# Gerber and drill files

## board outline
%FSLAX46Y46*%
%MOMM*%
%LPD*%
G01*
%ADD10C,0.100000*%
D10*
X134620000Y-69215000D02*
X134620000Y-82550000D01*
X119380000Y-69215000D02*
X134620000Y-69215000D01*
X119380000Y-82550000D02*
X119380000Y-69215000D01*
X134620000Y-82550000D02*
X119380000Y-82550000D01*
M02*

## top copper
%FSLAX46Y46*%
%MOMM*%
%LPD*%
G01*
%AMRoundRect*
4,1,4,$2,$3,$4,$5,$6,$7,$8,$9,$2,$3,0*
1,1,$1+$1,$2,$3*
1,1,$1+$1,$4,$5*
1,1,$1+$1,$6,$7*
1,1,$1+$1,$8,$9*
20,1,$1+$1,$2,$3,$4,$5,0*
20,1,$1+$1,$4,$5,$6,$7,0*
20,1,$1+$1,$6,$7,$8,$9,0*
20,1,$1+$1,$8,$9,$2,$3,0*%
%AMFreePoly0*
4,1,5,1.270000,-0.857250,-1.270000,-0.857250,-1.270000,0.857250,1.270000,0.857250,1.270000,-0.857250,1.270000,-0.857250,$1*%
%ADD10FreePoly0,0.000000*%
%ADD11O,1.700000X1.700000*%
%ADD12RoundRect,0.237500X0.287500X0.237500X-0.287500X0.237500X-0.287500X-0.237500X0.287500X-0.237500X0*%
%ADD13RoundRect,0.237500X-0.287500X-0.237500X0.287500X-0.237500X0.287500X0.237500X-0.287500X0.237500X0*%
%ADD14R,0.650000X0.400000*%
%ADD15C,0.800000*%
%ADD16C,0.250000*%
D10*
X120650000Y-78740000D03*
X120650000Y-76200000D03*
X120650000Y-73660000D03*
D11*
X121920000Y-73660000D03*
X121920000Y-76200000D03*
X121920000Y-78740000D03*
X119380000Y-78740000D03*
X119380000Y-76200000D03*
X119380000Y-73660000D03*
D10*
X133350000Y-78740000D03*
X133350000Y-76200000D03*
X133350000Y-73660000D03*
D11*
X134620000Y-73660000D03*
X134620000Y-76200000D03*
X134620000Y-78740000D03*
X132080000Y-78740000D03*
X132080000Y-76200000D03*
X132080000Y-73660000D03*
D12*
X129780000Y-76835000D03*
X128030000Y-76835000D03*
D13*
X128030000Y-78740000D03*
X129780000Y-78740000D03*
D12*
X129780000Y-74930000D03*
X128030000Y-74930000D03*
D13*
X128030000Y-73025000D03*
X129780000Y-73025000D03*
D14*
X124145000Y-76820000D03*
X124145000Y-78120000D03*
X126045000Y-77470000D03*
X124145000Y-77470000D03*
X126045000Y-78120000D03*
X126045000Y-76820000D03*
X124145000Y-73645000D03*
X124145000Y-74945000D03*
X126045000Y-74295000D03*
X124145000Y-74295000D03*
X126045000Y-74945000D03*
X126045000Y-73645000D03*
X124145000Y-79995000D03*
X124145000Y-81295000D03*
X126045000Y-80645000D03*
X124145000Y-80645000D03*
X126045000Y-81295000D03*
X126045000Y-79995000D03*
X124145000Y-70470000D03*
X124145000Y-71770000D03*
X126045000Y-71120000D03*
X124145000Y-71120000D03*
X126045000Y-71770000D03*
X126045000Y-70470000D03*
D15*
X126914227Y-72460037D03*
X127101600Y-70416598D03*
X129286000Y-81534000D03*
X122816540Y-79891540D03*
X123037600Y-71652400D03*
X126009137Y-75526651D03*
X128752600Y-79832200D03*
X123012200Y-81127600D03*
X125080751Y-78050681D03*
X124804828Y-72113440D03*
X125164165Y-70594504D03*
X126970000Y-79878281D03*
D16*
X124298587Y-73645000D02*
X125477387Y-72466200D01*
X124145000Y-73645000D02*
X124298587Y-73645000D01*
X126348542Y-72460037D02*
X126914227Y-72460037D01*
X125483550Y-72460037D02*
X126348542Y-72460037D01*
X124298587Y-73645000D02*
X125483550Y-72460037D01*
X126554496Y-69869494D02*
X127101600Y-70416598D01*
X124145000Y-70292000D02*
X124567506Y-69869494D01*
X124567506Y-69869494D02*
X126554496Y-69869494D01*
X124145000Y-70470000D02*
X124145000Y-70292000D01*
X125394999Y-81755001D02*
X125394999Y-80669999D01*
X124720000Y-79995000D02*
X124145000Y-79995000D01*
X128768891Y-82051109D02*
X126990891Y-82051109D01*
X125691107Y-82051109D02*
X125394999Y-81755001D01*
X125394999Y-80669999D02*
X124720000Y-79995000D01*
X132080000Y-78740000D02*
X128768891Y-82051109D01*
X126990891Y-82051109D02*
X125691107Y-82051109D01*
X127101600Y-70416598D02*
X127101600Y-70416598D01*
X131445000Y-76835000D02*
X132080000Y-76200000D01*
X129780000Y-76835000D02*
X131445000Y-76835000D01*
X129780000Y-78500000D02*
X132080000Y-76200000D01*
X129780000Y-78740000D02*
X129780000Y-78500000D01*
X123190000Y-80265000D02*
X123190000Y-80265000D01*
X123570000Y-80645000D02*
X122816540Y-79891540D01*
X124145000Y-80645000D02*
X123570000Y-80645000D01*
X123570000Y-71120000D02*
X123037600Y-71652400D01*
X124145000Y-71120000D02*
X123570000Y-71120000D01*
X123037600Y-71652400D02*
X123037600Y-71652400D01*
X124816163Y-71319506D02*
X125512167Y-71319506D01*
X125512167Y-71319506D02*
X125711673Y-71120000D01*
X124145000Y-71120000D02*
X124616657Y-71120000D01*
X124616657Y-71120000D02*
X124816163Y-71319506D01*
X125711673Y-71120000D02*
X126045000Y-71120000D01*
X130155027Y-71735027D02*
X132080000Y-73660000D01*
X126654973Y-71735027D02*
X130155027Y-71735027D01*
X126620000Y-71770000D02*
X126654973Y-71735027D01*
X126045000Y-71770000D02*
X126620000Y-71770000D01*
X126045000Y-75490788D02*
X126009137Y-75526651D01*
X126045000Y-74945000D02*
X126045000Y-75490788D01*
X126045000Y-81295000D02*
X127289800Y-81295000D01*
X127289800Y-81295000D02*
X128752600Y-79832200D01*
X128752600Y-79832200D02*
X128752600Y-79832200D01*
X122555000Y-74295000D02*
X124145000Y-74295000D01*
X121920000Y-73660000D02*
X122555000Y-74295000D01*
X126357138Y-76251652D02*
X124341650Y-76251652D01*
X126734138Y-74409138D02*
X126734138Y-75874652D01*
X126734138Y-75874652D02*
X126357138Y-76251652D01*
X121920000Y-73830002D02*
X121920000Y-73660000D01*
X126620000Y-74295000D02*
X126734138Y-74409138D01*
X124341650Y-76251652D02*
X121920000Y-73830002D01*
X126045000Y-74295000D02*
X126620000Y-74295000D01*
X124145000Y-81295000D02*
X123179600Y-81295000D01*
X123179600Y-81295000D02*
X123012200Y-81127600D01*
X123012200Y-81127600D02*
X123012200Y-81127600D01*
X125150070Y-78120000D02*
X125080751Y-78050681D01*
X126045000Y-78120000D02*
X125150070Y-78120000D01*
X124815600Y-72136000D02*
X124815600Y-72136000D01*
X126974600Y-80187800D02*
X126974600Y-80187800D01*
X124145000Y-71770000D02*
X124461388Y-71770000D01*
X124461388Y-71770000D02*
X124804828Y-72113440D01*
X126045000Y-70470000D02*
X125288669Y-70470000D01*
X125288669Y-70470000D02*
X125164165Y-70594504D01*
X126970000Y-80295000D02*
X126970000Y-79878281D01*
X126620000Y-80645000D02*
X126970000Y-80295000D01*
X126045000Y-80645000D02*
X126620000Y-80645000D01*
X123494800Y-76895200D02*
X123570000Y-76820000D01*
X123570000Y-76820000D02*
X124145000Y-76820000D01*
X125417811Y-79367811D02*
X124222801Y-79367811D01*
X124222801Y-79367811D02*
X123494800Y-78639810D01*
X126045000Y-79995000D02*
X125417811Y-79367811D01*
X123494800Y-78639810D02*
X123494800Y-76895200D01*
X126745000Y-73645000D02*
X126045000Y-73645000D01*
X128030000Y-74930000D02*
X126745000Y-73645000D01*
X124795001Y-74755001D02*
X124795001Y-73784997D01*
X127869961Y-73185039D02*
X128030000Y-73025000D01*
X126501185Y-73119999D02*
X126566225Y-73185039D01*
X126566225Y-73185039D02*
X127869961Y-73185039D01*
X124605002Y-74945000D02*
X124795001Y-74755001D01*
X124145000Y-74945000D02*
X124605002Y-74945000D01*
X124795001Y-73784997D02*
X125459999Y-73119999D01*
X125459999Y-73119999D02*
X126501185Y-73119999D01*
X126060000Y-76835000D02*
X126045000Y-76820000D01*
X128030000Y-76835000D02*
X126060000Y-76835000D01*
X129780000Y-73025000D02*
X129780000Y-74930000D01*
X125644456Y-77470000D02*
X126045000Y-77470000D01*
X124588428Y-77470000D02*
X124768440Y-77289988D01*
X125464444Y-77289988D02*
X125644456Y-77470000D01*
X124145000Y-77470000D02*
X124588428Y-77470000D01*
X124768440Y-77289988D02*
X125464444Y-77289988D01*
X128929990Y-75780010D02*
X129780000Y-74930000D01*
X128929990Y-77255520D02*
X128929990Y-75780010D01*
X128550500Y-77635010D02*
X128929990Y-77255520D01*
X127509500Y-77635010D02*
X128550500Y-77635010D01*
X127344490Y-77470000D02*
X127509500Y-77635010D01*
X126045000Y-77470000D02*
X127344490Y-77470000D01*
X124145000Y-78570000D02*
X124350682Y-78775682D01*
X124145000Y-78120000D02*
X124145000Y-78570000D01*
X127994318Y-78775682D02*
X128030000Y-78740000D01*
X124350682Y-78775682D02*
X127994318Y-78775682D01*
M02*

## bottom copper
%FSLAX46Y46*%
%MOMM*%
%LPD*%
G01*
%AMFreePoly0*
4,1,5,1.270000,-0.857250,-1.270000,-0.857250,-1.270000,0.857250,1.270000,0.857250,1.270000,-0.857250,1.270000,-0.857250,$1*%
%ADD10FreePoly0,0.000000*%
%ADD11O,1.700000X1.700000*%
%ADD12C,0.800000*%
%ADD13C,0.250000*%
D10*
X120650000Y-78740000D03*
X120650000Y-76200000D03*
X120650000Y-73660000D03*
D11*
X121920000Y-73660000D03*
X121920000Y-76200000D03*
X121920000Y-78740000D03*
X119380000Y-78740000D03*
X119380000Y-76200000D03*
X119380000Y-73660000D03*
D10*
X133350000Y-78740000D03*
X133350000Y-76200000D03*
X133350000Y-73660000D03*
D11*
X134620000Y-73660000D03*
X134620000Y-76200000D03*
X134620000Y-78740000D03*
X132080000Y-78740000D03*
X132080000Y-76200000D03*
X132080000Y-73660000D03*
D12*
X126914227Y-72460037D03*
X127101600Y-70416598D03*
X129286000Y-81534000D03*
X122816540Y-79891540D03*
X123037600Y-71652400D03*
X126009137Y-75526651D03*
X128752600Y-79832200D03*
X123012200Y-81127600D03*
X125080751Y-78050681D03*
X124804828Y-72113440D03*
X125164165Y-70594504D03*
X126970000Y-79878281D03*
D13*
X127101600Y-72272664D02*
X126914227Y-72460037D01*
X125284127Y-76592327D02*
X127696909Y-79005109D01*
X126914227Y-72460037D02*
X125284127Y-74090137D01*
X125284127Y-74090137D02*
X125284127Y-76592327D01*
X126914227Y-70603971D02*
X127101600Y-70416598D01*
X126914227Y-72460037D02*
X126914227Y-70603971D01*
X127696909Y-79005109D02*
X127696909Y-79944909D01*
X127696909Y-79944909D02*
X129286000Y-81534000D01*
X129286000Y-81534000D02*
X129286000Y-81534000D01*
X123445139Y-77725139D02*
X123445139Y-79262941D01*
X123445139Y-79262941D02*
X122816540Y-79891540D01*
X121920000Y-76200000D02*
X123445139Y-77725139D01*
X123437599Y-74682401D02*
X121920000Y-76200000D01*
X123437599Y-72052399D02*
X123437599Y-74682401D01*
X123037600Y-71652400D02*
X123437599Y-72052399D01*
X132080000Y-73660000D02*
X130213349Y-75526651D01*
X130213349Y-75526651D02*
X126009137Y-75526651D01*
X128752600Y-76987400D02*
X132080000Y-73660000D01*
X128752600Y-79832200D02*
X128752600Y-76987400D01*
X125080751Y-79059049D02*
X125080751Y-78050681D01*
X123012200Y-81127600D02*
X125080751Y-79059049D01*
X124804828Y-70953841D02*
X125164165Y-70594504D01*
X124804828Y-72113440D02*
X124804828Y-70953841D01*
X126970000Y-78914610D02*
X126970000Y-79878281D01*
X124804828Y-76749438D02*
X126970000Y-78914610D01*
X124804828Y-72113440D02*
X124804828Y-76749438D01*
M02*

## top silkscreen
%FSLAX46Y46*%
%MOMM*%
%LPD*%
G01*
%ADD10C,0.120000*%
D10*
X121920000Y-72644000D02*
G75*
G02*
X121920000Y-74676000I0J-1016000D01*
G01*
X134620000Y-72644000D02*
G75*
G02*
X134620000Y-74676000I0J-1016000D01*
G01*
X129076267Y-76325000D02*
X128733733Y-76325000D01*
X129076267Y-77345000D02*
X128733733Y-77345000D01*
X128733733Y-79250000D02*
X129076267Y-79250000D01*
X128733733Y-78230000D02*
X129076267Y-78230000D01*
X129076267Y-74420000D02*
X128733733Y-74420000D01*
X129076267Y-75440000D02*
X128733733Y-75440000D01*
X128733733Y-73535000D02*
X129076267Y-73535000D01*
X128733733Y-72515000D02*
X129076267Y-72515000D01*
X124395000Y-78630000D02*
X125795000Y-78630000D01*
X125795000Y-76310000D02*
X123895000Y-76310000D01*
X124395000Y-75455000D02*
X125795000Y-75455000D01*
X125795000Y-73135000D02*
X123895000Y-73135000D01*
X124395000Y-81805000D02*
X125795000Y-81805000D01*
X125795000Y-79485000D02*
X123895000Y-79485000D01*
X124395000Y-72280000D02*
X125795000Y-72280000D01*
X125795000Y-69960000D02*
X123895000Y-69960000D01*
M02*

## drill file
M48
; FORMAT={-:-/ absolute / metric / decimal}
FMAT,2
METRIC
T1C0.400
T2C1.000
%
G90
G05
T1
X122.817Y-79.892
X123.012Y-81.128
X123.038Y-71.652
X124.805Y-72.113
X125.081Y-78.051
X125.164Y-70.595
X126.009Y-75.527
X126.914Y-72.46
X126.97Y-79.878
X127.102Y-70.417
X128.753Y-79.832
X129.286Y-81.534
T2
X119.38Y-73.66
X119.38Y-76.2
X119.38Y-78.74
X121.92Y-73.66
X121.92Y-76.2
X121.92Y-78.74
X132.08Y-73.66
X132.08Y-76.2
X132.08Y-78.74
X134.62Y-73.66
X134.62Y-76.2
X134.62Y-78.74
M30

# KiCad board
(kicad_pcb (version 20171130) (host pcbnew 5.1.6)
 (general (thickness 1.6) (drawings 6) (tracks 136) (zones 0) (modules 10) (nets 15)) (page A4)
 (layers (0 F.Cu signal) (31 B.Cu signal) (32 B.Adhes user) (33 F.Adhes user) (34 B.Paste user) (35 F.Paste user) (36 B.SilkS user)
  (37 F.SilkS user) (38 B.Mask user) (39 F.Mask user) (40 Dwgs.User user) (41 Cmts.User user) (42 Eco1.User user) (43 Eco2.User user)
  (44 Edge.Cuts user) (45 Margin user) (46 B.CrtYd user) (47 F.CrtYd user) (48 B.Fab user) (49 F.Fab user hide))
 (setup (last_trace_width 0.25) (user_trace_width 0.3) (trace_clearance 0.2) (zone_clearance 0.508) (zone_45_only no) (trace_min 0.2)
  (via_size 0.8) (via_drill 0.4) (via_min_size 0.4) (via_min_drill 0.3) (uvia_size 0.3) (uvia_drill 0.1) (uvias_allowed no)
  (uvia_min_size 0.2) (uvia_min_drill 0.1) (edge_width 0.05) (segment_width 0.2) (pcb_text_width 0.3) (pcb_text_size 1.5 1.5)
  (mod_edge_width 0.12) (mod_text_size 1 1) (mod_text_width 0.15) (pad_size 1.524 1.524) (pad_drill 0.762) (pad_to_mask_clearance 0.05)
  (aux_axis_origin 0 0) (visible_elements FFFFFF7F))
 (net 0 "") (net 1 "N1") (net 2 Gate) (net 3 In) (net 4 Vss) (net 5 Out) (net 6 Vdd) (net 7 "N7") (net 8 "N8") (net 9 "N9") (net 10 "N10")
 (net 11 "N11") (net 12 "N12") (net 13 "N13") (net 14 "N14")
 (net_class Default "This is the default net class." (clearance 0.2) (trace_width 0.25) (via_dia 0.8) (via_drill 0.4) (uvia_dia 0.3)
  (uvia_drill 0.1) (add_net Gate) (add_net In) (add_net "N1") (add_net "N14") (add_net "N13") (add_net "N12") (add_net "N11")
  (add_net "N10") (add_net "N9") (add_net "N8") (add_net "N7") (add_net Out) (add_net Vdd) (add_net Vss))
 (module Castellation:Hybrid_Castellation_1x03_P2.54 (layer F.Cu) (at 120.65 73.66)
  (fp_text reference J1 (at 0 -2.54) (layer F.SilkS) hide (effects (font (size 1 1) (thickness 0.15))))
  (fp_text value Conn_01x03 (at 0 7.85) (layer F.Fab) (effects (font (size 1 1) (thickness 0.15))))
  (fp_arc (start 1.27 0) (end 1.27 1.016) (angle -180) (layer F.SilkS) (width 0.12))
  (pad 3 connect custom (at 0 5.08) (size 2.54 1.7145) (layers B.Cu B.Mask) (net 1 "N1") (zone_connect 0)
   (options (clearance outline) (anchor rect)) (primitives))
  (pad 2 connect custom (at 0 2.54) (size 2.54 1.7145) (layers B.Cu B.Mask) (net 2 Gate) (zone_connect 0)
   (options (clearance outline) (anchor rect)) (primitives))
  (pad 1 connect custom (at 0 0) (size 2.54 1.7145) (layers B.Cu B.Mask) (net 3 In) (zone_connect 0)
   (options (clearance outline) (anchor rect)) (primitives))
  (pad 3 connect custom (at 0 5.08) (size 2.54 1.7145) (layers F.Cu F.Mask) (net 1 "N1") (zone_connect 0)
   (options (clearance outline) (anchor rect)) (primitives))
  (pad 2 connect custom (at 0 2.54) (size 2.54 1.7145) (layers F.Cu F.Mask) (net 2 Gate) (zone_connect 0)
   (options (clearance outline) (anchor rect)) (primitives))
  (pad 1 connect custom (at 0 0) (size 2.54 1.7145) (layers F.Cu F.Mask) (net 3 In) (zone_connect 0)
   (options (clearance outline) (anchor rect)) (primitives))
  (pad 1 thru_hole oval (at 1.27 0) (size 1.7 1.7) (drill 1) (layers *.Cu *.Mask) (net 3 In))
  (pad 2 thru_hole oval (at 1.27 2.54) (size 1.7 1.7) (drill 1) (layers *.Cu *.Mask) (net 2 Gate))
  (pad 3 thru_hole oval (at 1.27 5.08) (size 1.7 1.7) (drill 1) (layers *.Cu *.Mask) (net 1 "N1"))
  (pad 3 thru_hole oval (at -1.27 5.08) (size 1.7 1.7) (drill 1) (layers *.Cu *.Mask) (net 1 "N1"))
  (pad 2 thru_hole oval (at -1.27 2.54) (size 1.7 1.7) (drill 1) (layers *.Cu *.Mask) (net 2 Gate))
  (pad 1 thru_hole oval (at -1.27 0) (size 1.7 1.7) (drill 1) (layers *.Cu *.Mask) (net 3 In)))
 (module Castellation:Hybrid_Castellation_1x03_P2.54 (layer F.Cu) (at 133.35 73.66)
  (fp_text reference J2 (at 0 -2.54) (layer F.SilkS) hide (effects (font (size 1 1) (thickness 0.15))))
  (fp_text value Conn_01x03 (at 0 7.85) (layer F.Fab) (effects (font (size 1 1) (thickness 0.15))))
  (fp_arc (start 1.27 0) (end 1.27 1.016) (angle -180) (layer F.SilkS) (width 0.12))
  (pad 3 connect custom (at 0 5.08) (size 2.54 1.7145) (layers B.Cu B.Mask) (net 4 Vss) (zone_connect 0)
   (options (clearance outline) (anchor rect)) (primitives))
  (pad 2 connect custom (at 0 2.54) (size 2.54 1.7145) (layers B.Cu B.Mask) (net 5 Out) (zone_connect 0)
   (options (clearance outline) (anchor rect)) (primitives))
  (pad 1 connect custom (at 0 0) (size 2.54 1.7145) (layers B.Cu B.Mask) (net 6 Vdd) (zone_connect 0)
   (options (clearance outline) (anchor rect)) (primitives))
  (pad 3 connect custom (at 0 5.08) (size 2.54 1.7145) (layers F.Cu F.Mask) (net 4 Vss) (zone_connect 0)
   (options (clearance outline) (anchor rect)) (primitives))
  (pad 2 connect custom (at 0 2.54) (size 2.54 1.7145) (layers F.Cu F.Mask) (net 5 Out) (zone_connect 0)
   (options (clearance outline) (anchor rect)) (primitives))
  (pad 1 connect custom (at 0 0) (size 2.54 1.7145) (layers F.Cu F.Mask) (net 6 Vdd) (zone_connect 0)
   (options (clearance outline) (anchor rect)) (primitives))
  (pad 1 thru_hole oval (at 1.27 0) (size 1.7 1.7) (drill 1) (layers *.Cu *.Mask) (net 6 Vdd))
  (pad 2 thru_hole oval (at 1.27 2.54) (size 1.7 1.7) (drill 1) (layers *.Cu *.Mask) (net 5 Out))
  (pad 3 thru_hole oval (at 1.27 5.08) (size 1.7 1.7) (drill 1) (layers *.Cu *.Mask) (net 4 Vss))
  (pad 3 thru_hole oval (at -1.27 5.08) (size 1.7 1.7) (drill 1) (layers *.Cu *.Mask) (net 4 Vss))
  (pad 2 thru_hole oval (at -1.27 2.54) (size 1.7 1.7) (drill 1) (layers *.Cu *.Mask) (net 5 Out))
  (pad 1 thru_hole oval (at -1.27 0) (size 1.7 1.7) (drill 1) (layers *.Cu *.Mask) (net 6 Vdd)))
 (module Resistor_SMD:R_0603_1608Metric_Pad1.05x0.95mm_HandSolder (layer F.Cu) (at 128.905 76.835 180)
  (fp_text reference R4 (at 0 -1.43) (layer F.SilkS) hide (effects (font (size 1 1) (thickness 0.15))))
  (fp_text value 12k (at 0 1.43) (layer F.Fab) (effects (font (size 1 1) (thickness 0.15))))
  (fp_line (start -0.171267 0.51) (end 0.171267 0.51) (layer F.SilkS) (width 0.12))
  (fp_line (start -0.171267 -0.51) (end 0.171267 -0.51) (layer F.SilkS) (width 0.12))
  (pad 1 smd roundrect (at -0.875 0 180) (size 1.05 0.95) (layers F.Cu F.Paste F.Mask) (roundrect_rratio 0.25) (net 5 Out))
  (pad 2 smd roundrect (at 0.875 0 180) (size 1.05 0.95) (layers F.Cu F.Paste F.Mask) (roundrect_rratio 0.25) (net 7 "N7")))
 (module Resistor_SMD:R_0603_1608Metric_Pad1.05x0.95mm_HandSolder (layer F.Cu) (at 128.905 78.74)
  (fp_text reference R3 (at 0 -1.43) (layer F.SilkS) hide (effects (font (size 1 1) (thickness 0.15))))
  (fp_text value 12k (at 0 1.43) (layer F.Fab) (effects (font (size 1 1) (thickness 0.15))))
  (fp_line (start -0.171267 0.51) (end 0.171267 0.51) (layer F.SilkS) (width 0.12))
  (fp_line (start -0.171267 -0.51) (end 0.171267 -0.51) (layer F.SilkS) (width 0.12))
  (pad 1 smd roundrect (at -0.875 0) (size 1.05 0.95) (layers F.Cu F.Paste F.Mask) (roundrect_rratio 0.25) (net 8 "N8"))
  (pad 2 smd roundrect (at 0.875 0) (size 1.05 0.95) (layers F.Cu F.Paste F.Mask) (roundrect_rratio 0.25) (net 5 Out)))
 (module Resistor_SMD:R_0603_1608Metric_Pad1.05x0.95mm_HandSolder (layer F.Cu) (at 128.905 74.93 180)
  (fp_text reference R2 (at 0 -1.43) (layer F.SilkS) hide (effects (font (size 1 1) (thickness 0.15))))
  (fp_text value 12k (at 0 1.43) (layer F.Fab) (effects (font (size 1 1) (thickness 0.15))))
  (fp_line (start -0.171267 0.51) (end 0.171267 0.51) (layer F.SilkS) (width 0.12))
  (fp_line (start -0.171267 -0.51) (end 0.171267 -0.51) (layer F.SilkS) (width 0.12))
  (pad 1 smd roundrect (at -0.875 0 180) (size 1.05 0.95) (layers F.Cu F.Paste F.Mask) (roundrect_rratio 0.25) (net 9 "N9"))
  (pad 2 smd roundrect (at 0.875 0 180) (size 1.05 0.95) (layers F.Cu F.Paste F.Mask) (roundrect_rratio 0.25) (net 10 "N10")))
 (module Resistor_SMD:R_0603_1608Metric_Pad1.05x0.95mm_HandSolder (layer F.Cu) (at 128.905 73.025)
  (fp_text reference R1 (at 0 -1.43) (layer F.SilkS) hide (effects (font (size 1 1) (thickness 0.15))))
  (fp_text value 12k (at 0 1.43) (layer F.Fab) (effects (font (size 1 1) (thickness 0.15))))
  (fp_line (start -0.171267 0.51) (end 0.171267 0.51) (layer F.SilkS) (width 0.12))
  (fp_line (start -0.171267 -0.51) (end 0.171267 -0.51) (layer F.SilkS) (width 0.12))
  (pad 1 smd roundrect (at -0.875 0) (size 1.05 0.95) (layers F.Cu F.Paste F.Mask) (roundrect_rratio 0.25) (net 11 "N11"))
  (pad 2 smd roundrect (at 0.875 0) (size 1.05 0.95) (layers F.Cu F.Paste F.Mask) (roundrect_rratio 0.25) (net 9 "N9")))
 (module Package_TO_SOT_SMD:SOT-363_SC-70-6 (layer F.Cu) (at 125.095 77.47)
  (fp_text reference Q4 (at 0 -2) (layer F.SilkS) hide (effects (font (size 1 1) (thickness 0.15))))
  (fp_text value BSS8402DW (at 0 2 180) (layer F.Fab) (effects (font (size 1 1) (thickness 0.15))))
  (fp_line (start -0.7 1.16) (end 0.7 1.16) (layer F.SilkS) (width 0.12))
  (fp_line (start 0.7 -1.16) (end -1.2 -1.16) (layer F.SilkS) (width 0.12))
  (pad 1 smd rect (at -0.95 -0.65) (size 0.65 0.4) (layers F.Cu F.Paste F.Mask) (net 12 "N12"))
  (pad 3 smd rect (at -0.95 0.65) (size 0.65 0.4) (layers F.Cu F.Paste F.Mask) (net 8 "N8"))
  (pad 5 smd rect (at 0.95 0) (size 0.65 0.4) (layers F.Cu F.Paste F.Mask) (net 9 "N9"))
  (pad 2 smd rect (at -0.95 0) (size 0.65 0.4) (layers F.Cu F.Paste F.Mask) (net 9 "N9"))
  (pad 4 smd rect (at 0.95 0.65) (size 0.65 0.4) (layers F.Cu F.Paste F.Mask) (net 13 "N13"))
  (pad 6 smd rect (at 0.95 -0.65) (size 0.65 0.4) (layers F.Cu F.Paste F.Mask) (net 7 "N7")))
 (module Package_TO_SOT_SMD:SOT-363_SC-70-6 (layer F.Cu) (at 125.095 74.295)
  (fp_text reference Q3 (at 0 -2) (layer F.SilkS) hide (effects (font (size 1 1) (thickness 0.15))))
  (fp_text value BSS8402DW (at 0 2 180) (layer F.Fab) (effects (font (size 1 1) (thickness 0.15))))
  (fp_line (start -0.7 1.16) (end 0.7 1.16) (layer F.SilkS) (width 0.12))
  (fp_line (start 0.7 -1.16) (end -1.2 -1.16) (layer F.SilkS) (width 0.12))
  (pad 1 smd rect (at -0.95 -0.65) (size 0.65 0.4) (layers F.Cu F.Paste F.Mask) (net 4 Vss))
  (pad 3 smd rect (at -0.95 0.65) (size 0.65 0.4) (layers F.Cu F.Paste F.Mask) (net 11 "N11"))
  (pad 5 smd rect (at 0.95 0) (size 0.65 0.4) (layers F.Cu F.Paste F.Mask) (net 3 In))
  (pad 2 smd rect (at -0.95 0) (size 0.65 0.4) (layers F.Cu F.Paste F.Mask) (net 3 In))
  (pad 4 smd rect (at 0.95 0.65) (size 0.65 0.4) (layers F.Cu F.Paste F.Mask) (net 6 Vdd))
  (pad 6 smd rect (at 0.95 -0.65) (size 0.65 0.4) (layers F.Cu F.Paste F.Mask) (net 10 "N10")))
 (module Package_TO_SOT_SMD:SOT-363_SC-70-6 (layer F.Cu) (at 125.095 80.645)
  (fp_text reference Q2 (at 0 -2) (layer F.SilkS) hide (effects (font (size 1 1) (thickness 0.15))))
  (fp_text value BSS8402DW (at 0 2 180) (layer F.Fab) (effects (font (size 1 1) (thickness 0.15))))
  (fp_line (start -0.7 1.16) (end 0.7 1.16) (layer F.SilkS) (width 0.12))
  (fp_line (start 0.7 -1.16) (end -1.2 -1.16) (layer F.SilkS) (width 0.12))
  (pad 1 smd rect (at -0.95 -0.65) (size 0.65 0.4) (layers F.Cu F.Paste F.Mask) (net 4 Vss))
  (pad 3 smd rect (at -0.95 0.65) (size 0.65 0.4) (layers F.Cu F.Paste F.Mask) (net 13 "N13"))
  (pad 5 smd rect (at 0.95 0) (size 0.65 0.4) (layers F.Cu F.Paste F.Mask) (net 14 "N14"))
  (pad 2 smd rect (at -0.95 0) (size 0.65 0.4) (layers F.Cu F.Paste F.Mask) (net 2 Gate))
  (pad 4 smd rect (at 0.95 0.65) (size 0.65 0.4) (layers F.Cu F.Paste F.Mask) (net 6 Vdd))
  (pad 6 smd rect (at 0.95 -0.65) (size 0.65 0.4) (layers F.Cu F.Paste F.Mask) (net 12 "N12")))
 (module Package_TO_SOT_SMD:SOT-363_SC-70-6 (layer F.Cu) (at 125.095 71.12)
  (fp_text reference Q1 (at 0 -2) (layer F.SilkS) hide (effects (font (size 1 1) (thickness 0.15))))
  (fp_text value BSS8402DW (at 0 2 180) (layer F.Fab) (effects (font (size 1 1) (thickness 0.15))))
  (fp_line (start -0.7 1.16) (end 0.7 1.16) (layer F.SilkS) (width 0.12))
  (fp_line (start 0.7 -1.16) (end -1.2 -1.16) (layer F.SilkS) (width 0.12))
  (pad 1 smd rect (at -0.95 -0.65) (size 0.65 0.4) (layers F.Cu F.Paste F.Mask) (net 4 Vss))
  (pad 3 smd rect (at -0.95 0.65) (size 0.65 0.4) (layers F.Cu F.Paste F.Mask) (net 14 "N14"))
  (pad 5 smd rect (at 0.95 0) (size 0.65 0.4) (layers F.Cu F.Paste F.Mask) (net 2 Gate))
  (pad 2 smd rect (at -0.95 0) (size 0.65 0.4) (layers F.Cu F.Paste F.Mask) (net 2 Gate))
  (pad 4 smd rect (at 0.95 0.65) (size 0.65 0.4) (layers F.Cu F.Paste F.Mask) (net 6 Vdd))
  (pad 6 smd rect (at 0.95 -0.65) (size 0.65 0.4) (layers F.Cu F.Paste F.Mask) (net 14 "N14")))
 (gr_line (start 134.62 69.215) (end 134.62 82.55) (layer Edge.Cuts) (width 0.1))
 (gr_line (start 119.38 69.215) (end 134.62 69.215) (layer Edge.Cuts) (width 0.1))
 (gr_line (start 119.38 82.55) (end 119.38 69.215) (layer Edge.Cuts) (width 0.1))
 (gr_line (start 134.62 82.55) (end 119.38 82.55) (layer Edge.Cuts) (width 0.1))
 (segment (start 124.298587 73.645) (end 125.477387 72.4662) (width 0.25) (layer F.Cu) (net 4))
 (segment (start 124.145 73.645) (end 124.298587 73.645) (width 0.25) (layer F.Cu) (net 4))
 (segment (start 126.348542 72.460037) (end 126.914227 72.460037) (width 0.25) (layer F.Cu) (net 4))
 (segment (start 125.48355 72.460037) (end 126.348542 72.460037) (width 0.25) (layer F.Cu) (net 4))
 (via (at 126.914227 72.460037) (size 0.8) (drill 0.4) (layers F.Cu B.Cu) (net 4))
 (segment (start 124.298587 73.645) (end 125.48355 72.460037) (width 0.25) (layer F.Cu) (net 4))
 (segment (start 126.554496 69.869494) (end 127.1016 70.416598) (width 0.25) (layer F.Cu) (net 4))
 (segment (start 124.145 70.292) (end 124.567506 69.869494) (width 0.25) (layer F.Cu) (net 4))
 (segment (start 124.567506 69.869494) (end 126.554496 69.869494) (width 0.25) (layer F.Cu) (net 4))
 (segment (start 124.145 70.47) (end 124.145 70.292) (width 0.25) (layer F.Cu) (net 4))
 (segment (start 127.1016 72.272664) (end 126.914227 72.460037) (width 0.25) (layer B.Cu) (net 4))
 (segment (start 125.394999 81.755001) (end 125.394999 80.669999) (width 0.25) (layer F.Cu) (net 4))
 (segment (start 124.72 79.995) (end 124.145 79.995) (width 0.25) (layer F.Cu) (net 4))
 (segment (start 128.768891 82.051109) (end 126.990891 82.051109) (width 0.25) (layer F.Cu) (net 4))
 (segment (start 125.691107 82.051109) (end 125.394999 81.755001) (width 0.25) (layer F.Cu) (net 4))
 (segment (start 125.394999 80.669999) (end 124.72 79.995) (width 0.25) (layer F.Cu) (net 4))
 (segment (start 132.08 78.74) (end 128.768891 82.051109) (width 0.25) (layer F.Cu) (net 4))
 (segment (start 126.990891 82.051109) (end 125.691107 82.051109) (width 0.25) (layer F.Cu) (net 4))
 (segment (start 125.284127 76.592327) (end 127.696909 79.005109) (width 0.25) (layer B.Cu) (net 4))
 (segment (start 126.914227 72.460037) (end 125.284127 74.090137) (width 0.25) (layer B.Cu) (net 4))
 (segment (start 125.284127 74.090137) (end 125.284127 76.592327) (width 0.25) (layer B.Cu) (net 4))
 (segment (start 127.1016 70.416598) (end 127.1016 70.416598) (width 0.25) (layer F.Cu) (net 4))
 (via (at 127.1016 70.416598) (size 0.8) (drill 0.4) (layers F.Cu B.Cu) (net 4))
 (segment (start 126.914227 70.603971) (end 127.1016 70.416598) (width 0.25) (layer B.Cu) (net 4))
 (segment (start 126.914227 72.460037) (end 126.914227 70.603971) (width 0.25) (layer B.Cu) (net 4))
 (segment (start 127.696909 79.005109) (end 127.696909 79.944909) (width 0.25) (layer B.Cu) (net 4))
 (segment (start 127.696909 79.944909) (end 129.286 81.534) (width 0.25) (layer B.Cu) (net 4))
 (segment (start 129.286 81.534) (end 129.286 81.534) (width 0.25) (layer B.Cu) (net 4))
 (via (at 129.286 81.534) (size 0.8) (drill 0.4) (layers F.Cu B.Cu) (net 4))
 (segment (start 131.445 76.835) (end 132.08 76.2) (width 0.25) (layer F.Cu) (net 5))
 (segment (start 129.78 76.835) (end 131.445 76.835) (width 0.25) (layer F.Cu) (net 5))
 (segment (start 129.78 78.5) (end 132.08 76.2) (width 0.25) (layer F.Cu) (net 5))
 (segment (start 129.78 78.74) (end 129.78 78.5) (width 0.25) (layer F.Cu) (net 5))
 (segment (start 123.19 80.265) (end 123.19 80.265) (width 0.25) (layer F.Cu) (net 2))
 (segment (start 123.445139 77.725139) (end 123.445139 79.262941) (width 0.25) (layer B.Cu) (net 2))
 (segment (start 123.57 80.645) (end 122.81654 79.89154) (width 0.25) (layer F.Cu) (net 2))
 (segment (start 124.145 80.645) (end 123.57 80.645) (width 0.25) (layer F.Cu) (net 2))
 (segment (start 123.445139 79.262941) (end 122.81654 79.89154) (width 0.25) (layer B.Cu) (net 2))
 (via (at 122.81654 79.89154) (size 0.8) (drill 0.4) (layers F.Cu B.Cu) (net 2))
 (segment (start 121.92 76.2) (end 123.445139 77.725139) (width 0.25) (layer B.Cu) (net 2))
 (segment (start 123.57 71.12) (end 123.0376 71.6524) (width 0.25) (layer F.Cu) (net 2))
 (segment (start 124.145 71.12) (end 123.57 71.12) (width 0.25) (layer F.Cu) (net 2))
 (segment (start 123.0376 71.6524) (end 123.0376 71.6524) (width 0.25) (layer F.Cu) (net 2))
 (via (at 123.0376 71.6524) (size 0.8) (drill 0.4) (layers F.Cu B.Cu) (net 2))
 (segment (start 123.437599 74.682401) (end 121.92 76.2) (width 0.25) (layer B.Cu) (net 2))
 (segment (start 123.437599 72.052399) (end 123.437599 74.682401) (width 0.25) (layer B.Cu) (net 2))
 (segment (start 123.0376 71.6524) (end 123.437599 72.052399) (width 0.25) (layer B.Cu) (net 2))
 (segment (start 124.816163 71.319506) (end 125.512167 71.319506) (width 0.25) (layer F.Cu) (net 2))
 (segment (start 125.512167 71.319506) (end 125.711673 71.12) (width 0.25) (layer F.Cu) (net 2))
 (segment (start 124.145 71.12) (end 124.616657 71.12) (width 0.25) (layer F.Cu) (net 2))
 (segment (start 124.616657 71.12) (end 124.816163 71.319506) (width 0.25) (layer F.Cu) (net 2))
 (segment (start 125.711673 71.12) (end 126.045 71.12) (width 0.25) (layer F.Cu) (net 2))
 (segment (start 130.155027 71.735027) (end 132.08 73.66) (width 0.25) (layer F.Cu) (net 6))
 (segment (start 126.654973 71.735027) (end 130.155027 71.735027) (width 0.25) (layer F.Cu) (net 6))
 (segment (start 126.62 71.77) (end 126.654973 71.735027) (width 0.25) (layer F.Cu) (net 6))
 (segment (start 126.045 71.77) (end 126.62 71.77) (width 0.25) (layer F.Cu) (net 6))
 (via (at 126.009137 75.526651) (size 0.8) (drill 0.4) (layers F.Cu B.Cu) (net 6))
 (segment (start 132.08 73.66) (end 130.213349 75.526651) (width 0.25) (layer B.Cu) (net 6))
 (segment (start 130.213349 75.526651) (end 126.009137 75.526651) (width 0.25) (layer B.Cu) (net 6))
 (segment (start 126.045 75.490788) (end 126.009137 75.526651) (width 0.25) (layer F.Cu) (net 6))
 (segment (start 126.045 74.945) (end 126.045 75.490788) (width 0.25) (layer F.Cu) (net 6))
 (segment (start 126.045 81.295) (end 127.2898 81.295) (width 0.25) (layer F.Cu) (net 6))
 (segment (start 127.2898 81.295) (end 128.7526 79.8322) (width 0.25) (layer F.Cu) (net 6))
 (segment (start 128.7526 79.8322) (end 128.7526 79.8322) (width 0.25) (layer F.Cu) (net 6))
 (via (at 128.7526 79.8322) (size 0.8) (drill 0.4) (layers F.Cu B.Cu) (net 6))
 (segment (start 128.7526 76.9874) (end 132.08 73.66) (width 0.25) (layer B.Cu) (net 6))
 (segment (start 128.7526 79.8322) (end 128.7526 76.9874) (width 0.25) (layer B.Cu) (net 6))
 (segment (start 122.555 74.295) (end 124.145 74.295) (width 0.25) (layer F.Cu) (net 3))
 (segment (start 121.92 73.66) (end 122.555 74.295) (width 0.25) (layer F.Cu) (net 3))
 (segment (start 126.357138 76.251652) (end 124.34165 76.251652) (width 0.25) (layer F.Cu) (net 3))
 (segment (start 126.734138 74.409138) (end 126.734138 75.874652) (width 0.25) (layer F.Cu) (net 3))
 (segment (start 126.734138 75.874652) (end 126.357138 76.251652) (width 0.25) (layer F.Cu) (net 3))
 (segment (start 121.92 73.830002) (end 121.92 73.66) (width 0.25) (layer F.Cu) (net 3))
 (segment (start 126.62 74.295) (end 126.734138 74.409138) (width 0.25) (layer F.Cu) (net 3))
 (segment (start 124.34165 76.251652) (end 121.92 73.830002) (width 0.25) (layer F.Cu) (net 3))
 (segment (start 126.045 74.295) (end 126.62 74.295) (width 0.25) (layer F.Cu) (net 3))
 (segment (start 124.145 81.295) (end 123.1796 81.295) (width 0.25) (layer F.Cu) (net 13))
 (segment (start 123.1796 81.295) (end 123.0122 81.1276) (width 0.25) (layer F.Cu) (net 13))
 (segment (start 123.0122 81.1276) (end 123.0122 81.1276) (width 0.25) (layer F.Cu) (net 13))
 (via (at 123.0122 81.1276) (size 0.8) (drill 0.4) (layers F.Cu B.Cu) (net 13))
 (segment (start 125.15007 78.12) (end 125.080751 78.050681) (width 0.25) (layer F.Cu) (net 13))
 (via (at 125.080751 78.050681) (size 0.8) (drill 0.4) (layers F.Cu B.Cu) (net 13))
 (segment (start 125.080751 79.059049) (end 125.080751 78.050681) (width 0.25) (layer B.Cu) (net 13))
 (segment (start 123.0122 81.1276) (end 125.080751 79.059049) (width 0.25) (layer B.Cu) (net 13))
 (segment (start 126.045 78.12) (end 125.15007 78.12) (width 0.25) (layer F.Cu) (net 13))
 (segment (start 124.8156 72.136) (end 124.8156 72.136) (width 0.25) (layer F.Cu) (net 14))
 (segment (start 126.9746 80.1878) (end 126.9746 80.1878) (width 0.25) (layer F.Cu) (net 14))
 (via (at 124.804828 72.11344) (size 0.8) (drill 0.4) (layers F.Cu B.Cu) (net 14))
 (segment (start 124.145 71.77) (end 124.461388 71.77) (width 0.25) (layer F.Cu) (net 14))
 (segment (start 124.461388 71.77) (end 124.804828 72.11344) (width 0.25) (layer F.Cu) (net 14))
 (segment (start 126.045 70.47) (end 125.288669 70.47) (width 0.25) (layer F.Cu) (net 14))
 (segment (start 124.804828 70.953841) (end 125.164165 70.594504) (width 0.25) (layer B.Cu) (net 14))
 (segment (start 124.804828 72.11344) (end 124.804828 70.953841) (width 0.25) (layer B.Cu) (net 14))
 (segment (start 125.288669 70.47) (end 125.164165 70.594504) (width 0.25) (layer F.Cu) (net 14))
 (via (at 125.164165 70.594504) (size 0.8) (drill 0.4) (layers F.Cu B.Cu) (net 14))
 (segment (start 126.97 78.91461) (end 126.97 79.878281) (width 0.25) (layer B.Cu) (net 14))
 (via (at 126.97 79.878281) (size 0.8) (drill 0.4) (layers F.Cu B.Cu) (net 14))
 (segment (start 126.97 80.295) (end 126.97 79.878281) (width 0.25) (layer F.Cu) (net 14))
 (segment (start 124.804828 76.749438) (end 126.97 78.91461) (width 0.25) (layer B.Cu) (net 14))
 (segment (start 124.804828 72.11344) (end 124.804828 76.749438) (width 0.25) (layer B.Cu) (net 14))
 (segment (start 126.62 80.645) (end 126.97 80.295) (width 0.25) (layer F.Cu) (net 14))
 (segment (start 126.045 80.645) (end 126.62 80.645) (width 0.25) (layer F.Cu) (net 14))
 (segment (start 123.4948 76.8952) (end 123.57 76.82) (width 0.25) (layer F.Cu) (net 12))
 (segment (start 123.57 76.82) (end 124.145 76.82) (width 0.25) (layer F.Cu) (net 12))
 (segment (start 125.417811 79.367811) (end 124.222801 79.367811) (width 0.25) (layer F.Cu) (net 12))
 (segment (start 124.222801 79.367811) (end 123.4948 78.63981) (width 0.25) (layer F.Cu) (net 12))
 (segment (start 126.045 79.995) (end 125.417811 79.367811) (width 0.25) (layer F.Cu) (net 12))
 (segment (start 123.4948 78.63981) (end 123.4948 76.8952) (width 0.25) (layer F.Cu) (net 12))
 (segment (start 126.745 73.645) (end 126.045 73.645) (width 0.25) (layer F.Cu) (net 10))
 (segment (start 128.03 74.93) (end 126.745 73.645) (width 0.25) (layer F.Cu) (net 10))
 (segment (start 124.795001 74.755001) (end 124.795001 73.784997) (width 0.25) (layer F.Cu) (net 11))
 (segment (start 127.869961 73.185039) (end 128.03 73.025) (width 0.25) (layer F.Cu) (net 11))
 (segment (start 126.501185 73.119999) (end 126.566225 73.185039) (width 0.25) (layer F.Cu) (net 11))
 (segment (start 126.566225 73.185039) (end 127.869961 73.185039) (width 0.25) (layer F.Cu) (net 11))
 (segment (start 124.605002 74.945) (end 124.795001 74.755001) (width 0.25) (layer F.Cu) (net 11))
 (segment (start 124.145 74.945) (end 124.605002 74.945) (width 0.25) (layer F.Cu) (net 11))
 (segment (start 124.795001 73.784997) (end 125.459999 73.119999) (width 0.25) (layer F.Cu) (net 11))
 (segment (start 125.459999 73.119999) (end 126.501185 73.119999) (width 0.25) (layer F.Cu) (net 11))
 (segment (start 126.06 76.835) (end 126.045 76.82) (width 0.25) (layer F.Cu) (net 7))
 (segment (start 128.03 76.835) (end 126.06 76.835) (width 0.25) (layer F.Cu) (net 7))
 (segment (start 129.78 73.025) (end 129.78 74.93) (width 0.25) (layer F.Cu) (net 9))
 (segment (start 125.644456 77.47) (end 126.045 77.47) (width 0.25) (layer F.Cu) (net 9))
 (segment (start 124.588428 77.47) (end 124.76844 77.289988) (width 0.25) (layer F.Cu) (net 9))
 (segment (start 125.464444 77.289988) (end 125.644456 77.47) (width 0.25) (layer F.Cu) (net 9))
 (segment (start 124.145 77.47) (end 124.588428 77.47) (width 0.25) (layer F.Cu) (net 9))
 (segment (start 124.76844 77.289988) (end 125.464444 77.289988) (width 0.25) (layer F.Cu) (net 9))
 (segment (start 128.92999 75.78001) (end 129.78 74.93) (width 0.25) (layer F.Cu) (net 9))
 (segment (start 128.92999 77.25552) (end 128.92999 75.78001) (width 0.25) (layer F.Cu) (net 9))
 (segment (start 128.5505 77.63501) (end 128.92999 77.25552) (width 0.25) (layer F.Cu) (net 9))
 (segment (start 127.5095 77.63501) (end 128.5505 77.63501) (width 0.25) (layer F.Cu) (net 9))
 (segment (start 127.34449 77.47) (end 127.5095 77.63501) (width 0.25) (layer F.Cu) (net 9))
 (segment (start 126.045 77.47) (end 127.34449 77.47) (width 0.25) (layer F.Cu) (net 9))
 (segment (start 124.145 78.57) (end 124.350682 78.775682) (width 0.25) (layer F.Cu) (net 8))
 (segment (start 124.145 78.12) (end 124.145 78.57) (width 0.25) (layer F.Cu) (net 8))
 (segment (start 127.994318 78.775682) (end 128.03 78.74) (width 0.25) (layer F.Cu) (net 8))
 (segment (start 124.350682 78.775682) (end 127.994318 78.775682) (width 0.25) (layer F.Cu) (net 8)))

